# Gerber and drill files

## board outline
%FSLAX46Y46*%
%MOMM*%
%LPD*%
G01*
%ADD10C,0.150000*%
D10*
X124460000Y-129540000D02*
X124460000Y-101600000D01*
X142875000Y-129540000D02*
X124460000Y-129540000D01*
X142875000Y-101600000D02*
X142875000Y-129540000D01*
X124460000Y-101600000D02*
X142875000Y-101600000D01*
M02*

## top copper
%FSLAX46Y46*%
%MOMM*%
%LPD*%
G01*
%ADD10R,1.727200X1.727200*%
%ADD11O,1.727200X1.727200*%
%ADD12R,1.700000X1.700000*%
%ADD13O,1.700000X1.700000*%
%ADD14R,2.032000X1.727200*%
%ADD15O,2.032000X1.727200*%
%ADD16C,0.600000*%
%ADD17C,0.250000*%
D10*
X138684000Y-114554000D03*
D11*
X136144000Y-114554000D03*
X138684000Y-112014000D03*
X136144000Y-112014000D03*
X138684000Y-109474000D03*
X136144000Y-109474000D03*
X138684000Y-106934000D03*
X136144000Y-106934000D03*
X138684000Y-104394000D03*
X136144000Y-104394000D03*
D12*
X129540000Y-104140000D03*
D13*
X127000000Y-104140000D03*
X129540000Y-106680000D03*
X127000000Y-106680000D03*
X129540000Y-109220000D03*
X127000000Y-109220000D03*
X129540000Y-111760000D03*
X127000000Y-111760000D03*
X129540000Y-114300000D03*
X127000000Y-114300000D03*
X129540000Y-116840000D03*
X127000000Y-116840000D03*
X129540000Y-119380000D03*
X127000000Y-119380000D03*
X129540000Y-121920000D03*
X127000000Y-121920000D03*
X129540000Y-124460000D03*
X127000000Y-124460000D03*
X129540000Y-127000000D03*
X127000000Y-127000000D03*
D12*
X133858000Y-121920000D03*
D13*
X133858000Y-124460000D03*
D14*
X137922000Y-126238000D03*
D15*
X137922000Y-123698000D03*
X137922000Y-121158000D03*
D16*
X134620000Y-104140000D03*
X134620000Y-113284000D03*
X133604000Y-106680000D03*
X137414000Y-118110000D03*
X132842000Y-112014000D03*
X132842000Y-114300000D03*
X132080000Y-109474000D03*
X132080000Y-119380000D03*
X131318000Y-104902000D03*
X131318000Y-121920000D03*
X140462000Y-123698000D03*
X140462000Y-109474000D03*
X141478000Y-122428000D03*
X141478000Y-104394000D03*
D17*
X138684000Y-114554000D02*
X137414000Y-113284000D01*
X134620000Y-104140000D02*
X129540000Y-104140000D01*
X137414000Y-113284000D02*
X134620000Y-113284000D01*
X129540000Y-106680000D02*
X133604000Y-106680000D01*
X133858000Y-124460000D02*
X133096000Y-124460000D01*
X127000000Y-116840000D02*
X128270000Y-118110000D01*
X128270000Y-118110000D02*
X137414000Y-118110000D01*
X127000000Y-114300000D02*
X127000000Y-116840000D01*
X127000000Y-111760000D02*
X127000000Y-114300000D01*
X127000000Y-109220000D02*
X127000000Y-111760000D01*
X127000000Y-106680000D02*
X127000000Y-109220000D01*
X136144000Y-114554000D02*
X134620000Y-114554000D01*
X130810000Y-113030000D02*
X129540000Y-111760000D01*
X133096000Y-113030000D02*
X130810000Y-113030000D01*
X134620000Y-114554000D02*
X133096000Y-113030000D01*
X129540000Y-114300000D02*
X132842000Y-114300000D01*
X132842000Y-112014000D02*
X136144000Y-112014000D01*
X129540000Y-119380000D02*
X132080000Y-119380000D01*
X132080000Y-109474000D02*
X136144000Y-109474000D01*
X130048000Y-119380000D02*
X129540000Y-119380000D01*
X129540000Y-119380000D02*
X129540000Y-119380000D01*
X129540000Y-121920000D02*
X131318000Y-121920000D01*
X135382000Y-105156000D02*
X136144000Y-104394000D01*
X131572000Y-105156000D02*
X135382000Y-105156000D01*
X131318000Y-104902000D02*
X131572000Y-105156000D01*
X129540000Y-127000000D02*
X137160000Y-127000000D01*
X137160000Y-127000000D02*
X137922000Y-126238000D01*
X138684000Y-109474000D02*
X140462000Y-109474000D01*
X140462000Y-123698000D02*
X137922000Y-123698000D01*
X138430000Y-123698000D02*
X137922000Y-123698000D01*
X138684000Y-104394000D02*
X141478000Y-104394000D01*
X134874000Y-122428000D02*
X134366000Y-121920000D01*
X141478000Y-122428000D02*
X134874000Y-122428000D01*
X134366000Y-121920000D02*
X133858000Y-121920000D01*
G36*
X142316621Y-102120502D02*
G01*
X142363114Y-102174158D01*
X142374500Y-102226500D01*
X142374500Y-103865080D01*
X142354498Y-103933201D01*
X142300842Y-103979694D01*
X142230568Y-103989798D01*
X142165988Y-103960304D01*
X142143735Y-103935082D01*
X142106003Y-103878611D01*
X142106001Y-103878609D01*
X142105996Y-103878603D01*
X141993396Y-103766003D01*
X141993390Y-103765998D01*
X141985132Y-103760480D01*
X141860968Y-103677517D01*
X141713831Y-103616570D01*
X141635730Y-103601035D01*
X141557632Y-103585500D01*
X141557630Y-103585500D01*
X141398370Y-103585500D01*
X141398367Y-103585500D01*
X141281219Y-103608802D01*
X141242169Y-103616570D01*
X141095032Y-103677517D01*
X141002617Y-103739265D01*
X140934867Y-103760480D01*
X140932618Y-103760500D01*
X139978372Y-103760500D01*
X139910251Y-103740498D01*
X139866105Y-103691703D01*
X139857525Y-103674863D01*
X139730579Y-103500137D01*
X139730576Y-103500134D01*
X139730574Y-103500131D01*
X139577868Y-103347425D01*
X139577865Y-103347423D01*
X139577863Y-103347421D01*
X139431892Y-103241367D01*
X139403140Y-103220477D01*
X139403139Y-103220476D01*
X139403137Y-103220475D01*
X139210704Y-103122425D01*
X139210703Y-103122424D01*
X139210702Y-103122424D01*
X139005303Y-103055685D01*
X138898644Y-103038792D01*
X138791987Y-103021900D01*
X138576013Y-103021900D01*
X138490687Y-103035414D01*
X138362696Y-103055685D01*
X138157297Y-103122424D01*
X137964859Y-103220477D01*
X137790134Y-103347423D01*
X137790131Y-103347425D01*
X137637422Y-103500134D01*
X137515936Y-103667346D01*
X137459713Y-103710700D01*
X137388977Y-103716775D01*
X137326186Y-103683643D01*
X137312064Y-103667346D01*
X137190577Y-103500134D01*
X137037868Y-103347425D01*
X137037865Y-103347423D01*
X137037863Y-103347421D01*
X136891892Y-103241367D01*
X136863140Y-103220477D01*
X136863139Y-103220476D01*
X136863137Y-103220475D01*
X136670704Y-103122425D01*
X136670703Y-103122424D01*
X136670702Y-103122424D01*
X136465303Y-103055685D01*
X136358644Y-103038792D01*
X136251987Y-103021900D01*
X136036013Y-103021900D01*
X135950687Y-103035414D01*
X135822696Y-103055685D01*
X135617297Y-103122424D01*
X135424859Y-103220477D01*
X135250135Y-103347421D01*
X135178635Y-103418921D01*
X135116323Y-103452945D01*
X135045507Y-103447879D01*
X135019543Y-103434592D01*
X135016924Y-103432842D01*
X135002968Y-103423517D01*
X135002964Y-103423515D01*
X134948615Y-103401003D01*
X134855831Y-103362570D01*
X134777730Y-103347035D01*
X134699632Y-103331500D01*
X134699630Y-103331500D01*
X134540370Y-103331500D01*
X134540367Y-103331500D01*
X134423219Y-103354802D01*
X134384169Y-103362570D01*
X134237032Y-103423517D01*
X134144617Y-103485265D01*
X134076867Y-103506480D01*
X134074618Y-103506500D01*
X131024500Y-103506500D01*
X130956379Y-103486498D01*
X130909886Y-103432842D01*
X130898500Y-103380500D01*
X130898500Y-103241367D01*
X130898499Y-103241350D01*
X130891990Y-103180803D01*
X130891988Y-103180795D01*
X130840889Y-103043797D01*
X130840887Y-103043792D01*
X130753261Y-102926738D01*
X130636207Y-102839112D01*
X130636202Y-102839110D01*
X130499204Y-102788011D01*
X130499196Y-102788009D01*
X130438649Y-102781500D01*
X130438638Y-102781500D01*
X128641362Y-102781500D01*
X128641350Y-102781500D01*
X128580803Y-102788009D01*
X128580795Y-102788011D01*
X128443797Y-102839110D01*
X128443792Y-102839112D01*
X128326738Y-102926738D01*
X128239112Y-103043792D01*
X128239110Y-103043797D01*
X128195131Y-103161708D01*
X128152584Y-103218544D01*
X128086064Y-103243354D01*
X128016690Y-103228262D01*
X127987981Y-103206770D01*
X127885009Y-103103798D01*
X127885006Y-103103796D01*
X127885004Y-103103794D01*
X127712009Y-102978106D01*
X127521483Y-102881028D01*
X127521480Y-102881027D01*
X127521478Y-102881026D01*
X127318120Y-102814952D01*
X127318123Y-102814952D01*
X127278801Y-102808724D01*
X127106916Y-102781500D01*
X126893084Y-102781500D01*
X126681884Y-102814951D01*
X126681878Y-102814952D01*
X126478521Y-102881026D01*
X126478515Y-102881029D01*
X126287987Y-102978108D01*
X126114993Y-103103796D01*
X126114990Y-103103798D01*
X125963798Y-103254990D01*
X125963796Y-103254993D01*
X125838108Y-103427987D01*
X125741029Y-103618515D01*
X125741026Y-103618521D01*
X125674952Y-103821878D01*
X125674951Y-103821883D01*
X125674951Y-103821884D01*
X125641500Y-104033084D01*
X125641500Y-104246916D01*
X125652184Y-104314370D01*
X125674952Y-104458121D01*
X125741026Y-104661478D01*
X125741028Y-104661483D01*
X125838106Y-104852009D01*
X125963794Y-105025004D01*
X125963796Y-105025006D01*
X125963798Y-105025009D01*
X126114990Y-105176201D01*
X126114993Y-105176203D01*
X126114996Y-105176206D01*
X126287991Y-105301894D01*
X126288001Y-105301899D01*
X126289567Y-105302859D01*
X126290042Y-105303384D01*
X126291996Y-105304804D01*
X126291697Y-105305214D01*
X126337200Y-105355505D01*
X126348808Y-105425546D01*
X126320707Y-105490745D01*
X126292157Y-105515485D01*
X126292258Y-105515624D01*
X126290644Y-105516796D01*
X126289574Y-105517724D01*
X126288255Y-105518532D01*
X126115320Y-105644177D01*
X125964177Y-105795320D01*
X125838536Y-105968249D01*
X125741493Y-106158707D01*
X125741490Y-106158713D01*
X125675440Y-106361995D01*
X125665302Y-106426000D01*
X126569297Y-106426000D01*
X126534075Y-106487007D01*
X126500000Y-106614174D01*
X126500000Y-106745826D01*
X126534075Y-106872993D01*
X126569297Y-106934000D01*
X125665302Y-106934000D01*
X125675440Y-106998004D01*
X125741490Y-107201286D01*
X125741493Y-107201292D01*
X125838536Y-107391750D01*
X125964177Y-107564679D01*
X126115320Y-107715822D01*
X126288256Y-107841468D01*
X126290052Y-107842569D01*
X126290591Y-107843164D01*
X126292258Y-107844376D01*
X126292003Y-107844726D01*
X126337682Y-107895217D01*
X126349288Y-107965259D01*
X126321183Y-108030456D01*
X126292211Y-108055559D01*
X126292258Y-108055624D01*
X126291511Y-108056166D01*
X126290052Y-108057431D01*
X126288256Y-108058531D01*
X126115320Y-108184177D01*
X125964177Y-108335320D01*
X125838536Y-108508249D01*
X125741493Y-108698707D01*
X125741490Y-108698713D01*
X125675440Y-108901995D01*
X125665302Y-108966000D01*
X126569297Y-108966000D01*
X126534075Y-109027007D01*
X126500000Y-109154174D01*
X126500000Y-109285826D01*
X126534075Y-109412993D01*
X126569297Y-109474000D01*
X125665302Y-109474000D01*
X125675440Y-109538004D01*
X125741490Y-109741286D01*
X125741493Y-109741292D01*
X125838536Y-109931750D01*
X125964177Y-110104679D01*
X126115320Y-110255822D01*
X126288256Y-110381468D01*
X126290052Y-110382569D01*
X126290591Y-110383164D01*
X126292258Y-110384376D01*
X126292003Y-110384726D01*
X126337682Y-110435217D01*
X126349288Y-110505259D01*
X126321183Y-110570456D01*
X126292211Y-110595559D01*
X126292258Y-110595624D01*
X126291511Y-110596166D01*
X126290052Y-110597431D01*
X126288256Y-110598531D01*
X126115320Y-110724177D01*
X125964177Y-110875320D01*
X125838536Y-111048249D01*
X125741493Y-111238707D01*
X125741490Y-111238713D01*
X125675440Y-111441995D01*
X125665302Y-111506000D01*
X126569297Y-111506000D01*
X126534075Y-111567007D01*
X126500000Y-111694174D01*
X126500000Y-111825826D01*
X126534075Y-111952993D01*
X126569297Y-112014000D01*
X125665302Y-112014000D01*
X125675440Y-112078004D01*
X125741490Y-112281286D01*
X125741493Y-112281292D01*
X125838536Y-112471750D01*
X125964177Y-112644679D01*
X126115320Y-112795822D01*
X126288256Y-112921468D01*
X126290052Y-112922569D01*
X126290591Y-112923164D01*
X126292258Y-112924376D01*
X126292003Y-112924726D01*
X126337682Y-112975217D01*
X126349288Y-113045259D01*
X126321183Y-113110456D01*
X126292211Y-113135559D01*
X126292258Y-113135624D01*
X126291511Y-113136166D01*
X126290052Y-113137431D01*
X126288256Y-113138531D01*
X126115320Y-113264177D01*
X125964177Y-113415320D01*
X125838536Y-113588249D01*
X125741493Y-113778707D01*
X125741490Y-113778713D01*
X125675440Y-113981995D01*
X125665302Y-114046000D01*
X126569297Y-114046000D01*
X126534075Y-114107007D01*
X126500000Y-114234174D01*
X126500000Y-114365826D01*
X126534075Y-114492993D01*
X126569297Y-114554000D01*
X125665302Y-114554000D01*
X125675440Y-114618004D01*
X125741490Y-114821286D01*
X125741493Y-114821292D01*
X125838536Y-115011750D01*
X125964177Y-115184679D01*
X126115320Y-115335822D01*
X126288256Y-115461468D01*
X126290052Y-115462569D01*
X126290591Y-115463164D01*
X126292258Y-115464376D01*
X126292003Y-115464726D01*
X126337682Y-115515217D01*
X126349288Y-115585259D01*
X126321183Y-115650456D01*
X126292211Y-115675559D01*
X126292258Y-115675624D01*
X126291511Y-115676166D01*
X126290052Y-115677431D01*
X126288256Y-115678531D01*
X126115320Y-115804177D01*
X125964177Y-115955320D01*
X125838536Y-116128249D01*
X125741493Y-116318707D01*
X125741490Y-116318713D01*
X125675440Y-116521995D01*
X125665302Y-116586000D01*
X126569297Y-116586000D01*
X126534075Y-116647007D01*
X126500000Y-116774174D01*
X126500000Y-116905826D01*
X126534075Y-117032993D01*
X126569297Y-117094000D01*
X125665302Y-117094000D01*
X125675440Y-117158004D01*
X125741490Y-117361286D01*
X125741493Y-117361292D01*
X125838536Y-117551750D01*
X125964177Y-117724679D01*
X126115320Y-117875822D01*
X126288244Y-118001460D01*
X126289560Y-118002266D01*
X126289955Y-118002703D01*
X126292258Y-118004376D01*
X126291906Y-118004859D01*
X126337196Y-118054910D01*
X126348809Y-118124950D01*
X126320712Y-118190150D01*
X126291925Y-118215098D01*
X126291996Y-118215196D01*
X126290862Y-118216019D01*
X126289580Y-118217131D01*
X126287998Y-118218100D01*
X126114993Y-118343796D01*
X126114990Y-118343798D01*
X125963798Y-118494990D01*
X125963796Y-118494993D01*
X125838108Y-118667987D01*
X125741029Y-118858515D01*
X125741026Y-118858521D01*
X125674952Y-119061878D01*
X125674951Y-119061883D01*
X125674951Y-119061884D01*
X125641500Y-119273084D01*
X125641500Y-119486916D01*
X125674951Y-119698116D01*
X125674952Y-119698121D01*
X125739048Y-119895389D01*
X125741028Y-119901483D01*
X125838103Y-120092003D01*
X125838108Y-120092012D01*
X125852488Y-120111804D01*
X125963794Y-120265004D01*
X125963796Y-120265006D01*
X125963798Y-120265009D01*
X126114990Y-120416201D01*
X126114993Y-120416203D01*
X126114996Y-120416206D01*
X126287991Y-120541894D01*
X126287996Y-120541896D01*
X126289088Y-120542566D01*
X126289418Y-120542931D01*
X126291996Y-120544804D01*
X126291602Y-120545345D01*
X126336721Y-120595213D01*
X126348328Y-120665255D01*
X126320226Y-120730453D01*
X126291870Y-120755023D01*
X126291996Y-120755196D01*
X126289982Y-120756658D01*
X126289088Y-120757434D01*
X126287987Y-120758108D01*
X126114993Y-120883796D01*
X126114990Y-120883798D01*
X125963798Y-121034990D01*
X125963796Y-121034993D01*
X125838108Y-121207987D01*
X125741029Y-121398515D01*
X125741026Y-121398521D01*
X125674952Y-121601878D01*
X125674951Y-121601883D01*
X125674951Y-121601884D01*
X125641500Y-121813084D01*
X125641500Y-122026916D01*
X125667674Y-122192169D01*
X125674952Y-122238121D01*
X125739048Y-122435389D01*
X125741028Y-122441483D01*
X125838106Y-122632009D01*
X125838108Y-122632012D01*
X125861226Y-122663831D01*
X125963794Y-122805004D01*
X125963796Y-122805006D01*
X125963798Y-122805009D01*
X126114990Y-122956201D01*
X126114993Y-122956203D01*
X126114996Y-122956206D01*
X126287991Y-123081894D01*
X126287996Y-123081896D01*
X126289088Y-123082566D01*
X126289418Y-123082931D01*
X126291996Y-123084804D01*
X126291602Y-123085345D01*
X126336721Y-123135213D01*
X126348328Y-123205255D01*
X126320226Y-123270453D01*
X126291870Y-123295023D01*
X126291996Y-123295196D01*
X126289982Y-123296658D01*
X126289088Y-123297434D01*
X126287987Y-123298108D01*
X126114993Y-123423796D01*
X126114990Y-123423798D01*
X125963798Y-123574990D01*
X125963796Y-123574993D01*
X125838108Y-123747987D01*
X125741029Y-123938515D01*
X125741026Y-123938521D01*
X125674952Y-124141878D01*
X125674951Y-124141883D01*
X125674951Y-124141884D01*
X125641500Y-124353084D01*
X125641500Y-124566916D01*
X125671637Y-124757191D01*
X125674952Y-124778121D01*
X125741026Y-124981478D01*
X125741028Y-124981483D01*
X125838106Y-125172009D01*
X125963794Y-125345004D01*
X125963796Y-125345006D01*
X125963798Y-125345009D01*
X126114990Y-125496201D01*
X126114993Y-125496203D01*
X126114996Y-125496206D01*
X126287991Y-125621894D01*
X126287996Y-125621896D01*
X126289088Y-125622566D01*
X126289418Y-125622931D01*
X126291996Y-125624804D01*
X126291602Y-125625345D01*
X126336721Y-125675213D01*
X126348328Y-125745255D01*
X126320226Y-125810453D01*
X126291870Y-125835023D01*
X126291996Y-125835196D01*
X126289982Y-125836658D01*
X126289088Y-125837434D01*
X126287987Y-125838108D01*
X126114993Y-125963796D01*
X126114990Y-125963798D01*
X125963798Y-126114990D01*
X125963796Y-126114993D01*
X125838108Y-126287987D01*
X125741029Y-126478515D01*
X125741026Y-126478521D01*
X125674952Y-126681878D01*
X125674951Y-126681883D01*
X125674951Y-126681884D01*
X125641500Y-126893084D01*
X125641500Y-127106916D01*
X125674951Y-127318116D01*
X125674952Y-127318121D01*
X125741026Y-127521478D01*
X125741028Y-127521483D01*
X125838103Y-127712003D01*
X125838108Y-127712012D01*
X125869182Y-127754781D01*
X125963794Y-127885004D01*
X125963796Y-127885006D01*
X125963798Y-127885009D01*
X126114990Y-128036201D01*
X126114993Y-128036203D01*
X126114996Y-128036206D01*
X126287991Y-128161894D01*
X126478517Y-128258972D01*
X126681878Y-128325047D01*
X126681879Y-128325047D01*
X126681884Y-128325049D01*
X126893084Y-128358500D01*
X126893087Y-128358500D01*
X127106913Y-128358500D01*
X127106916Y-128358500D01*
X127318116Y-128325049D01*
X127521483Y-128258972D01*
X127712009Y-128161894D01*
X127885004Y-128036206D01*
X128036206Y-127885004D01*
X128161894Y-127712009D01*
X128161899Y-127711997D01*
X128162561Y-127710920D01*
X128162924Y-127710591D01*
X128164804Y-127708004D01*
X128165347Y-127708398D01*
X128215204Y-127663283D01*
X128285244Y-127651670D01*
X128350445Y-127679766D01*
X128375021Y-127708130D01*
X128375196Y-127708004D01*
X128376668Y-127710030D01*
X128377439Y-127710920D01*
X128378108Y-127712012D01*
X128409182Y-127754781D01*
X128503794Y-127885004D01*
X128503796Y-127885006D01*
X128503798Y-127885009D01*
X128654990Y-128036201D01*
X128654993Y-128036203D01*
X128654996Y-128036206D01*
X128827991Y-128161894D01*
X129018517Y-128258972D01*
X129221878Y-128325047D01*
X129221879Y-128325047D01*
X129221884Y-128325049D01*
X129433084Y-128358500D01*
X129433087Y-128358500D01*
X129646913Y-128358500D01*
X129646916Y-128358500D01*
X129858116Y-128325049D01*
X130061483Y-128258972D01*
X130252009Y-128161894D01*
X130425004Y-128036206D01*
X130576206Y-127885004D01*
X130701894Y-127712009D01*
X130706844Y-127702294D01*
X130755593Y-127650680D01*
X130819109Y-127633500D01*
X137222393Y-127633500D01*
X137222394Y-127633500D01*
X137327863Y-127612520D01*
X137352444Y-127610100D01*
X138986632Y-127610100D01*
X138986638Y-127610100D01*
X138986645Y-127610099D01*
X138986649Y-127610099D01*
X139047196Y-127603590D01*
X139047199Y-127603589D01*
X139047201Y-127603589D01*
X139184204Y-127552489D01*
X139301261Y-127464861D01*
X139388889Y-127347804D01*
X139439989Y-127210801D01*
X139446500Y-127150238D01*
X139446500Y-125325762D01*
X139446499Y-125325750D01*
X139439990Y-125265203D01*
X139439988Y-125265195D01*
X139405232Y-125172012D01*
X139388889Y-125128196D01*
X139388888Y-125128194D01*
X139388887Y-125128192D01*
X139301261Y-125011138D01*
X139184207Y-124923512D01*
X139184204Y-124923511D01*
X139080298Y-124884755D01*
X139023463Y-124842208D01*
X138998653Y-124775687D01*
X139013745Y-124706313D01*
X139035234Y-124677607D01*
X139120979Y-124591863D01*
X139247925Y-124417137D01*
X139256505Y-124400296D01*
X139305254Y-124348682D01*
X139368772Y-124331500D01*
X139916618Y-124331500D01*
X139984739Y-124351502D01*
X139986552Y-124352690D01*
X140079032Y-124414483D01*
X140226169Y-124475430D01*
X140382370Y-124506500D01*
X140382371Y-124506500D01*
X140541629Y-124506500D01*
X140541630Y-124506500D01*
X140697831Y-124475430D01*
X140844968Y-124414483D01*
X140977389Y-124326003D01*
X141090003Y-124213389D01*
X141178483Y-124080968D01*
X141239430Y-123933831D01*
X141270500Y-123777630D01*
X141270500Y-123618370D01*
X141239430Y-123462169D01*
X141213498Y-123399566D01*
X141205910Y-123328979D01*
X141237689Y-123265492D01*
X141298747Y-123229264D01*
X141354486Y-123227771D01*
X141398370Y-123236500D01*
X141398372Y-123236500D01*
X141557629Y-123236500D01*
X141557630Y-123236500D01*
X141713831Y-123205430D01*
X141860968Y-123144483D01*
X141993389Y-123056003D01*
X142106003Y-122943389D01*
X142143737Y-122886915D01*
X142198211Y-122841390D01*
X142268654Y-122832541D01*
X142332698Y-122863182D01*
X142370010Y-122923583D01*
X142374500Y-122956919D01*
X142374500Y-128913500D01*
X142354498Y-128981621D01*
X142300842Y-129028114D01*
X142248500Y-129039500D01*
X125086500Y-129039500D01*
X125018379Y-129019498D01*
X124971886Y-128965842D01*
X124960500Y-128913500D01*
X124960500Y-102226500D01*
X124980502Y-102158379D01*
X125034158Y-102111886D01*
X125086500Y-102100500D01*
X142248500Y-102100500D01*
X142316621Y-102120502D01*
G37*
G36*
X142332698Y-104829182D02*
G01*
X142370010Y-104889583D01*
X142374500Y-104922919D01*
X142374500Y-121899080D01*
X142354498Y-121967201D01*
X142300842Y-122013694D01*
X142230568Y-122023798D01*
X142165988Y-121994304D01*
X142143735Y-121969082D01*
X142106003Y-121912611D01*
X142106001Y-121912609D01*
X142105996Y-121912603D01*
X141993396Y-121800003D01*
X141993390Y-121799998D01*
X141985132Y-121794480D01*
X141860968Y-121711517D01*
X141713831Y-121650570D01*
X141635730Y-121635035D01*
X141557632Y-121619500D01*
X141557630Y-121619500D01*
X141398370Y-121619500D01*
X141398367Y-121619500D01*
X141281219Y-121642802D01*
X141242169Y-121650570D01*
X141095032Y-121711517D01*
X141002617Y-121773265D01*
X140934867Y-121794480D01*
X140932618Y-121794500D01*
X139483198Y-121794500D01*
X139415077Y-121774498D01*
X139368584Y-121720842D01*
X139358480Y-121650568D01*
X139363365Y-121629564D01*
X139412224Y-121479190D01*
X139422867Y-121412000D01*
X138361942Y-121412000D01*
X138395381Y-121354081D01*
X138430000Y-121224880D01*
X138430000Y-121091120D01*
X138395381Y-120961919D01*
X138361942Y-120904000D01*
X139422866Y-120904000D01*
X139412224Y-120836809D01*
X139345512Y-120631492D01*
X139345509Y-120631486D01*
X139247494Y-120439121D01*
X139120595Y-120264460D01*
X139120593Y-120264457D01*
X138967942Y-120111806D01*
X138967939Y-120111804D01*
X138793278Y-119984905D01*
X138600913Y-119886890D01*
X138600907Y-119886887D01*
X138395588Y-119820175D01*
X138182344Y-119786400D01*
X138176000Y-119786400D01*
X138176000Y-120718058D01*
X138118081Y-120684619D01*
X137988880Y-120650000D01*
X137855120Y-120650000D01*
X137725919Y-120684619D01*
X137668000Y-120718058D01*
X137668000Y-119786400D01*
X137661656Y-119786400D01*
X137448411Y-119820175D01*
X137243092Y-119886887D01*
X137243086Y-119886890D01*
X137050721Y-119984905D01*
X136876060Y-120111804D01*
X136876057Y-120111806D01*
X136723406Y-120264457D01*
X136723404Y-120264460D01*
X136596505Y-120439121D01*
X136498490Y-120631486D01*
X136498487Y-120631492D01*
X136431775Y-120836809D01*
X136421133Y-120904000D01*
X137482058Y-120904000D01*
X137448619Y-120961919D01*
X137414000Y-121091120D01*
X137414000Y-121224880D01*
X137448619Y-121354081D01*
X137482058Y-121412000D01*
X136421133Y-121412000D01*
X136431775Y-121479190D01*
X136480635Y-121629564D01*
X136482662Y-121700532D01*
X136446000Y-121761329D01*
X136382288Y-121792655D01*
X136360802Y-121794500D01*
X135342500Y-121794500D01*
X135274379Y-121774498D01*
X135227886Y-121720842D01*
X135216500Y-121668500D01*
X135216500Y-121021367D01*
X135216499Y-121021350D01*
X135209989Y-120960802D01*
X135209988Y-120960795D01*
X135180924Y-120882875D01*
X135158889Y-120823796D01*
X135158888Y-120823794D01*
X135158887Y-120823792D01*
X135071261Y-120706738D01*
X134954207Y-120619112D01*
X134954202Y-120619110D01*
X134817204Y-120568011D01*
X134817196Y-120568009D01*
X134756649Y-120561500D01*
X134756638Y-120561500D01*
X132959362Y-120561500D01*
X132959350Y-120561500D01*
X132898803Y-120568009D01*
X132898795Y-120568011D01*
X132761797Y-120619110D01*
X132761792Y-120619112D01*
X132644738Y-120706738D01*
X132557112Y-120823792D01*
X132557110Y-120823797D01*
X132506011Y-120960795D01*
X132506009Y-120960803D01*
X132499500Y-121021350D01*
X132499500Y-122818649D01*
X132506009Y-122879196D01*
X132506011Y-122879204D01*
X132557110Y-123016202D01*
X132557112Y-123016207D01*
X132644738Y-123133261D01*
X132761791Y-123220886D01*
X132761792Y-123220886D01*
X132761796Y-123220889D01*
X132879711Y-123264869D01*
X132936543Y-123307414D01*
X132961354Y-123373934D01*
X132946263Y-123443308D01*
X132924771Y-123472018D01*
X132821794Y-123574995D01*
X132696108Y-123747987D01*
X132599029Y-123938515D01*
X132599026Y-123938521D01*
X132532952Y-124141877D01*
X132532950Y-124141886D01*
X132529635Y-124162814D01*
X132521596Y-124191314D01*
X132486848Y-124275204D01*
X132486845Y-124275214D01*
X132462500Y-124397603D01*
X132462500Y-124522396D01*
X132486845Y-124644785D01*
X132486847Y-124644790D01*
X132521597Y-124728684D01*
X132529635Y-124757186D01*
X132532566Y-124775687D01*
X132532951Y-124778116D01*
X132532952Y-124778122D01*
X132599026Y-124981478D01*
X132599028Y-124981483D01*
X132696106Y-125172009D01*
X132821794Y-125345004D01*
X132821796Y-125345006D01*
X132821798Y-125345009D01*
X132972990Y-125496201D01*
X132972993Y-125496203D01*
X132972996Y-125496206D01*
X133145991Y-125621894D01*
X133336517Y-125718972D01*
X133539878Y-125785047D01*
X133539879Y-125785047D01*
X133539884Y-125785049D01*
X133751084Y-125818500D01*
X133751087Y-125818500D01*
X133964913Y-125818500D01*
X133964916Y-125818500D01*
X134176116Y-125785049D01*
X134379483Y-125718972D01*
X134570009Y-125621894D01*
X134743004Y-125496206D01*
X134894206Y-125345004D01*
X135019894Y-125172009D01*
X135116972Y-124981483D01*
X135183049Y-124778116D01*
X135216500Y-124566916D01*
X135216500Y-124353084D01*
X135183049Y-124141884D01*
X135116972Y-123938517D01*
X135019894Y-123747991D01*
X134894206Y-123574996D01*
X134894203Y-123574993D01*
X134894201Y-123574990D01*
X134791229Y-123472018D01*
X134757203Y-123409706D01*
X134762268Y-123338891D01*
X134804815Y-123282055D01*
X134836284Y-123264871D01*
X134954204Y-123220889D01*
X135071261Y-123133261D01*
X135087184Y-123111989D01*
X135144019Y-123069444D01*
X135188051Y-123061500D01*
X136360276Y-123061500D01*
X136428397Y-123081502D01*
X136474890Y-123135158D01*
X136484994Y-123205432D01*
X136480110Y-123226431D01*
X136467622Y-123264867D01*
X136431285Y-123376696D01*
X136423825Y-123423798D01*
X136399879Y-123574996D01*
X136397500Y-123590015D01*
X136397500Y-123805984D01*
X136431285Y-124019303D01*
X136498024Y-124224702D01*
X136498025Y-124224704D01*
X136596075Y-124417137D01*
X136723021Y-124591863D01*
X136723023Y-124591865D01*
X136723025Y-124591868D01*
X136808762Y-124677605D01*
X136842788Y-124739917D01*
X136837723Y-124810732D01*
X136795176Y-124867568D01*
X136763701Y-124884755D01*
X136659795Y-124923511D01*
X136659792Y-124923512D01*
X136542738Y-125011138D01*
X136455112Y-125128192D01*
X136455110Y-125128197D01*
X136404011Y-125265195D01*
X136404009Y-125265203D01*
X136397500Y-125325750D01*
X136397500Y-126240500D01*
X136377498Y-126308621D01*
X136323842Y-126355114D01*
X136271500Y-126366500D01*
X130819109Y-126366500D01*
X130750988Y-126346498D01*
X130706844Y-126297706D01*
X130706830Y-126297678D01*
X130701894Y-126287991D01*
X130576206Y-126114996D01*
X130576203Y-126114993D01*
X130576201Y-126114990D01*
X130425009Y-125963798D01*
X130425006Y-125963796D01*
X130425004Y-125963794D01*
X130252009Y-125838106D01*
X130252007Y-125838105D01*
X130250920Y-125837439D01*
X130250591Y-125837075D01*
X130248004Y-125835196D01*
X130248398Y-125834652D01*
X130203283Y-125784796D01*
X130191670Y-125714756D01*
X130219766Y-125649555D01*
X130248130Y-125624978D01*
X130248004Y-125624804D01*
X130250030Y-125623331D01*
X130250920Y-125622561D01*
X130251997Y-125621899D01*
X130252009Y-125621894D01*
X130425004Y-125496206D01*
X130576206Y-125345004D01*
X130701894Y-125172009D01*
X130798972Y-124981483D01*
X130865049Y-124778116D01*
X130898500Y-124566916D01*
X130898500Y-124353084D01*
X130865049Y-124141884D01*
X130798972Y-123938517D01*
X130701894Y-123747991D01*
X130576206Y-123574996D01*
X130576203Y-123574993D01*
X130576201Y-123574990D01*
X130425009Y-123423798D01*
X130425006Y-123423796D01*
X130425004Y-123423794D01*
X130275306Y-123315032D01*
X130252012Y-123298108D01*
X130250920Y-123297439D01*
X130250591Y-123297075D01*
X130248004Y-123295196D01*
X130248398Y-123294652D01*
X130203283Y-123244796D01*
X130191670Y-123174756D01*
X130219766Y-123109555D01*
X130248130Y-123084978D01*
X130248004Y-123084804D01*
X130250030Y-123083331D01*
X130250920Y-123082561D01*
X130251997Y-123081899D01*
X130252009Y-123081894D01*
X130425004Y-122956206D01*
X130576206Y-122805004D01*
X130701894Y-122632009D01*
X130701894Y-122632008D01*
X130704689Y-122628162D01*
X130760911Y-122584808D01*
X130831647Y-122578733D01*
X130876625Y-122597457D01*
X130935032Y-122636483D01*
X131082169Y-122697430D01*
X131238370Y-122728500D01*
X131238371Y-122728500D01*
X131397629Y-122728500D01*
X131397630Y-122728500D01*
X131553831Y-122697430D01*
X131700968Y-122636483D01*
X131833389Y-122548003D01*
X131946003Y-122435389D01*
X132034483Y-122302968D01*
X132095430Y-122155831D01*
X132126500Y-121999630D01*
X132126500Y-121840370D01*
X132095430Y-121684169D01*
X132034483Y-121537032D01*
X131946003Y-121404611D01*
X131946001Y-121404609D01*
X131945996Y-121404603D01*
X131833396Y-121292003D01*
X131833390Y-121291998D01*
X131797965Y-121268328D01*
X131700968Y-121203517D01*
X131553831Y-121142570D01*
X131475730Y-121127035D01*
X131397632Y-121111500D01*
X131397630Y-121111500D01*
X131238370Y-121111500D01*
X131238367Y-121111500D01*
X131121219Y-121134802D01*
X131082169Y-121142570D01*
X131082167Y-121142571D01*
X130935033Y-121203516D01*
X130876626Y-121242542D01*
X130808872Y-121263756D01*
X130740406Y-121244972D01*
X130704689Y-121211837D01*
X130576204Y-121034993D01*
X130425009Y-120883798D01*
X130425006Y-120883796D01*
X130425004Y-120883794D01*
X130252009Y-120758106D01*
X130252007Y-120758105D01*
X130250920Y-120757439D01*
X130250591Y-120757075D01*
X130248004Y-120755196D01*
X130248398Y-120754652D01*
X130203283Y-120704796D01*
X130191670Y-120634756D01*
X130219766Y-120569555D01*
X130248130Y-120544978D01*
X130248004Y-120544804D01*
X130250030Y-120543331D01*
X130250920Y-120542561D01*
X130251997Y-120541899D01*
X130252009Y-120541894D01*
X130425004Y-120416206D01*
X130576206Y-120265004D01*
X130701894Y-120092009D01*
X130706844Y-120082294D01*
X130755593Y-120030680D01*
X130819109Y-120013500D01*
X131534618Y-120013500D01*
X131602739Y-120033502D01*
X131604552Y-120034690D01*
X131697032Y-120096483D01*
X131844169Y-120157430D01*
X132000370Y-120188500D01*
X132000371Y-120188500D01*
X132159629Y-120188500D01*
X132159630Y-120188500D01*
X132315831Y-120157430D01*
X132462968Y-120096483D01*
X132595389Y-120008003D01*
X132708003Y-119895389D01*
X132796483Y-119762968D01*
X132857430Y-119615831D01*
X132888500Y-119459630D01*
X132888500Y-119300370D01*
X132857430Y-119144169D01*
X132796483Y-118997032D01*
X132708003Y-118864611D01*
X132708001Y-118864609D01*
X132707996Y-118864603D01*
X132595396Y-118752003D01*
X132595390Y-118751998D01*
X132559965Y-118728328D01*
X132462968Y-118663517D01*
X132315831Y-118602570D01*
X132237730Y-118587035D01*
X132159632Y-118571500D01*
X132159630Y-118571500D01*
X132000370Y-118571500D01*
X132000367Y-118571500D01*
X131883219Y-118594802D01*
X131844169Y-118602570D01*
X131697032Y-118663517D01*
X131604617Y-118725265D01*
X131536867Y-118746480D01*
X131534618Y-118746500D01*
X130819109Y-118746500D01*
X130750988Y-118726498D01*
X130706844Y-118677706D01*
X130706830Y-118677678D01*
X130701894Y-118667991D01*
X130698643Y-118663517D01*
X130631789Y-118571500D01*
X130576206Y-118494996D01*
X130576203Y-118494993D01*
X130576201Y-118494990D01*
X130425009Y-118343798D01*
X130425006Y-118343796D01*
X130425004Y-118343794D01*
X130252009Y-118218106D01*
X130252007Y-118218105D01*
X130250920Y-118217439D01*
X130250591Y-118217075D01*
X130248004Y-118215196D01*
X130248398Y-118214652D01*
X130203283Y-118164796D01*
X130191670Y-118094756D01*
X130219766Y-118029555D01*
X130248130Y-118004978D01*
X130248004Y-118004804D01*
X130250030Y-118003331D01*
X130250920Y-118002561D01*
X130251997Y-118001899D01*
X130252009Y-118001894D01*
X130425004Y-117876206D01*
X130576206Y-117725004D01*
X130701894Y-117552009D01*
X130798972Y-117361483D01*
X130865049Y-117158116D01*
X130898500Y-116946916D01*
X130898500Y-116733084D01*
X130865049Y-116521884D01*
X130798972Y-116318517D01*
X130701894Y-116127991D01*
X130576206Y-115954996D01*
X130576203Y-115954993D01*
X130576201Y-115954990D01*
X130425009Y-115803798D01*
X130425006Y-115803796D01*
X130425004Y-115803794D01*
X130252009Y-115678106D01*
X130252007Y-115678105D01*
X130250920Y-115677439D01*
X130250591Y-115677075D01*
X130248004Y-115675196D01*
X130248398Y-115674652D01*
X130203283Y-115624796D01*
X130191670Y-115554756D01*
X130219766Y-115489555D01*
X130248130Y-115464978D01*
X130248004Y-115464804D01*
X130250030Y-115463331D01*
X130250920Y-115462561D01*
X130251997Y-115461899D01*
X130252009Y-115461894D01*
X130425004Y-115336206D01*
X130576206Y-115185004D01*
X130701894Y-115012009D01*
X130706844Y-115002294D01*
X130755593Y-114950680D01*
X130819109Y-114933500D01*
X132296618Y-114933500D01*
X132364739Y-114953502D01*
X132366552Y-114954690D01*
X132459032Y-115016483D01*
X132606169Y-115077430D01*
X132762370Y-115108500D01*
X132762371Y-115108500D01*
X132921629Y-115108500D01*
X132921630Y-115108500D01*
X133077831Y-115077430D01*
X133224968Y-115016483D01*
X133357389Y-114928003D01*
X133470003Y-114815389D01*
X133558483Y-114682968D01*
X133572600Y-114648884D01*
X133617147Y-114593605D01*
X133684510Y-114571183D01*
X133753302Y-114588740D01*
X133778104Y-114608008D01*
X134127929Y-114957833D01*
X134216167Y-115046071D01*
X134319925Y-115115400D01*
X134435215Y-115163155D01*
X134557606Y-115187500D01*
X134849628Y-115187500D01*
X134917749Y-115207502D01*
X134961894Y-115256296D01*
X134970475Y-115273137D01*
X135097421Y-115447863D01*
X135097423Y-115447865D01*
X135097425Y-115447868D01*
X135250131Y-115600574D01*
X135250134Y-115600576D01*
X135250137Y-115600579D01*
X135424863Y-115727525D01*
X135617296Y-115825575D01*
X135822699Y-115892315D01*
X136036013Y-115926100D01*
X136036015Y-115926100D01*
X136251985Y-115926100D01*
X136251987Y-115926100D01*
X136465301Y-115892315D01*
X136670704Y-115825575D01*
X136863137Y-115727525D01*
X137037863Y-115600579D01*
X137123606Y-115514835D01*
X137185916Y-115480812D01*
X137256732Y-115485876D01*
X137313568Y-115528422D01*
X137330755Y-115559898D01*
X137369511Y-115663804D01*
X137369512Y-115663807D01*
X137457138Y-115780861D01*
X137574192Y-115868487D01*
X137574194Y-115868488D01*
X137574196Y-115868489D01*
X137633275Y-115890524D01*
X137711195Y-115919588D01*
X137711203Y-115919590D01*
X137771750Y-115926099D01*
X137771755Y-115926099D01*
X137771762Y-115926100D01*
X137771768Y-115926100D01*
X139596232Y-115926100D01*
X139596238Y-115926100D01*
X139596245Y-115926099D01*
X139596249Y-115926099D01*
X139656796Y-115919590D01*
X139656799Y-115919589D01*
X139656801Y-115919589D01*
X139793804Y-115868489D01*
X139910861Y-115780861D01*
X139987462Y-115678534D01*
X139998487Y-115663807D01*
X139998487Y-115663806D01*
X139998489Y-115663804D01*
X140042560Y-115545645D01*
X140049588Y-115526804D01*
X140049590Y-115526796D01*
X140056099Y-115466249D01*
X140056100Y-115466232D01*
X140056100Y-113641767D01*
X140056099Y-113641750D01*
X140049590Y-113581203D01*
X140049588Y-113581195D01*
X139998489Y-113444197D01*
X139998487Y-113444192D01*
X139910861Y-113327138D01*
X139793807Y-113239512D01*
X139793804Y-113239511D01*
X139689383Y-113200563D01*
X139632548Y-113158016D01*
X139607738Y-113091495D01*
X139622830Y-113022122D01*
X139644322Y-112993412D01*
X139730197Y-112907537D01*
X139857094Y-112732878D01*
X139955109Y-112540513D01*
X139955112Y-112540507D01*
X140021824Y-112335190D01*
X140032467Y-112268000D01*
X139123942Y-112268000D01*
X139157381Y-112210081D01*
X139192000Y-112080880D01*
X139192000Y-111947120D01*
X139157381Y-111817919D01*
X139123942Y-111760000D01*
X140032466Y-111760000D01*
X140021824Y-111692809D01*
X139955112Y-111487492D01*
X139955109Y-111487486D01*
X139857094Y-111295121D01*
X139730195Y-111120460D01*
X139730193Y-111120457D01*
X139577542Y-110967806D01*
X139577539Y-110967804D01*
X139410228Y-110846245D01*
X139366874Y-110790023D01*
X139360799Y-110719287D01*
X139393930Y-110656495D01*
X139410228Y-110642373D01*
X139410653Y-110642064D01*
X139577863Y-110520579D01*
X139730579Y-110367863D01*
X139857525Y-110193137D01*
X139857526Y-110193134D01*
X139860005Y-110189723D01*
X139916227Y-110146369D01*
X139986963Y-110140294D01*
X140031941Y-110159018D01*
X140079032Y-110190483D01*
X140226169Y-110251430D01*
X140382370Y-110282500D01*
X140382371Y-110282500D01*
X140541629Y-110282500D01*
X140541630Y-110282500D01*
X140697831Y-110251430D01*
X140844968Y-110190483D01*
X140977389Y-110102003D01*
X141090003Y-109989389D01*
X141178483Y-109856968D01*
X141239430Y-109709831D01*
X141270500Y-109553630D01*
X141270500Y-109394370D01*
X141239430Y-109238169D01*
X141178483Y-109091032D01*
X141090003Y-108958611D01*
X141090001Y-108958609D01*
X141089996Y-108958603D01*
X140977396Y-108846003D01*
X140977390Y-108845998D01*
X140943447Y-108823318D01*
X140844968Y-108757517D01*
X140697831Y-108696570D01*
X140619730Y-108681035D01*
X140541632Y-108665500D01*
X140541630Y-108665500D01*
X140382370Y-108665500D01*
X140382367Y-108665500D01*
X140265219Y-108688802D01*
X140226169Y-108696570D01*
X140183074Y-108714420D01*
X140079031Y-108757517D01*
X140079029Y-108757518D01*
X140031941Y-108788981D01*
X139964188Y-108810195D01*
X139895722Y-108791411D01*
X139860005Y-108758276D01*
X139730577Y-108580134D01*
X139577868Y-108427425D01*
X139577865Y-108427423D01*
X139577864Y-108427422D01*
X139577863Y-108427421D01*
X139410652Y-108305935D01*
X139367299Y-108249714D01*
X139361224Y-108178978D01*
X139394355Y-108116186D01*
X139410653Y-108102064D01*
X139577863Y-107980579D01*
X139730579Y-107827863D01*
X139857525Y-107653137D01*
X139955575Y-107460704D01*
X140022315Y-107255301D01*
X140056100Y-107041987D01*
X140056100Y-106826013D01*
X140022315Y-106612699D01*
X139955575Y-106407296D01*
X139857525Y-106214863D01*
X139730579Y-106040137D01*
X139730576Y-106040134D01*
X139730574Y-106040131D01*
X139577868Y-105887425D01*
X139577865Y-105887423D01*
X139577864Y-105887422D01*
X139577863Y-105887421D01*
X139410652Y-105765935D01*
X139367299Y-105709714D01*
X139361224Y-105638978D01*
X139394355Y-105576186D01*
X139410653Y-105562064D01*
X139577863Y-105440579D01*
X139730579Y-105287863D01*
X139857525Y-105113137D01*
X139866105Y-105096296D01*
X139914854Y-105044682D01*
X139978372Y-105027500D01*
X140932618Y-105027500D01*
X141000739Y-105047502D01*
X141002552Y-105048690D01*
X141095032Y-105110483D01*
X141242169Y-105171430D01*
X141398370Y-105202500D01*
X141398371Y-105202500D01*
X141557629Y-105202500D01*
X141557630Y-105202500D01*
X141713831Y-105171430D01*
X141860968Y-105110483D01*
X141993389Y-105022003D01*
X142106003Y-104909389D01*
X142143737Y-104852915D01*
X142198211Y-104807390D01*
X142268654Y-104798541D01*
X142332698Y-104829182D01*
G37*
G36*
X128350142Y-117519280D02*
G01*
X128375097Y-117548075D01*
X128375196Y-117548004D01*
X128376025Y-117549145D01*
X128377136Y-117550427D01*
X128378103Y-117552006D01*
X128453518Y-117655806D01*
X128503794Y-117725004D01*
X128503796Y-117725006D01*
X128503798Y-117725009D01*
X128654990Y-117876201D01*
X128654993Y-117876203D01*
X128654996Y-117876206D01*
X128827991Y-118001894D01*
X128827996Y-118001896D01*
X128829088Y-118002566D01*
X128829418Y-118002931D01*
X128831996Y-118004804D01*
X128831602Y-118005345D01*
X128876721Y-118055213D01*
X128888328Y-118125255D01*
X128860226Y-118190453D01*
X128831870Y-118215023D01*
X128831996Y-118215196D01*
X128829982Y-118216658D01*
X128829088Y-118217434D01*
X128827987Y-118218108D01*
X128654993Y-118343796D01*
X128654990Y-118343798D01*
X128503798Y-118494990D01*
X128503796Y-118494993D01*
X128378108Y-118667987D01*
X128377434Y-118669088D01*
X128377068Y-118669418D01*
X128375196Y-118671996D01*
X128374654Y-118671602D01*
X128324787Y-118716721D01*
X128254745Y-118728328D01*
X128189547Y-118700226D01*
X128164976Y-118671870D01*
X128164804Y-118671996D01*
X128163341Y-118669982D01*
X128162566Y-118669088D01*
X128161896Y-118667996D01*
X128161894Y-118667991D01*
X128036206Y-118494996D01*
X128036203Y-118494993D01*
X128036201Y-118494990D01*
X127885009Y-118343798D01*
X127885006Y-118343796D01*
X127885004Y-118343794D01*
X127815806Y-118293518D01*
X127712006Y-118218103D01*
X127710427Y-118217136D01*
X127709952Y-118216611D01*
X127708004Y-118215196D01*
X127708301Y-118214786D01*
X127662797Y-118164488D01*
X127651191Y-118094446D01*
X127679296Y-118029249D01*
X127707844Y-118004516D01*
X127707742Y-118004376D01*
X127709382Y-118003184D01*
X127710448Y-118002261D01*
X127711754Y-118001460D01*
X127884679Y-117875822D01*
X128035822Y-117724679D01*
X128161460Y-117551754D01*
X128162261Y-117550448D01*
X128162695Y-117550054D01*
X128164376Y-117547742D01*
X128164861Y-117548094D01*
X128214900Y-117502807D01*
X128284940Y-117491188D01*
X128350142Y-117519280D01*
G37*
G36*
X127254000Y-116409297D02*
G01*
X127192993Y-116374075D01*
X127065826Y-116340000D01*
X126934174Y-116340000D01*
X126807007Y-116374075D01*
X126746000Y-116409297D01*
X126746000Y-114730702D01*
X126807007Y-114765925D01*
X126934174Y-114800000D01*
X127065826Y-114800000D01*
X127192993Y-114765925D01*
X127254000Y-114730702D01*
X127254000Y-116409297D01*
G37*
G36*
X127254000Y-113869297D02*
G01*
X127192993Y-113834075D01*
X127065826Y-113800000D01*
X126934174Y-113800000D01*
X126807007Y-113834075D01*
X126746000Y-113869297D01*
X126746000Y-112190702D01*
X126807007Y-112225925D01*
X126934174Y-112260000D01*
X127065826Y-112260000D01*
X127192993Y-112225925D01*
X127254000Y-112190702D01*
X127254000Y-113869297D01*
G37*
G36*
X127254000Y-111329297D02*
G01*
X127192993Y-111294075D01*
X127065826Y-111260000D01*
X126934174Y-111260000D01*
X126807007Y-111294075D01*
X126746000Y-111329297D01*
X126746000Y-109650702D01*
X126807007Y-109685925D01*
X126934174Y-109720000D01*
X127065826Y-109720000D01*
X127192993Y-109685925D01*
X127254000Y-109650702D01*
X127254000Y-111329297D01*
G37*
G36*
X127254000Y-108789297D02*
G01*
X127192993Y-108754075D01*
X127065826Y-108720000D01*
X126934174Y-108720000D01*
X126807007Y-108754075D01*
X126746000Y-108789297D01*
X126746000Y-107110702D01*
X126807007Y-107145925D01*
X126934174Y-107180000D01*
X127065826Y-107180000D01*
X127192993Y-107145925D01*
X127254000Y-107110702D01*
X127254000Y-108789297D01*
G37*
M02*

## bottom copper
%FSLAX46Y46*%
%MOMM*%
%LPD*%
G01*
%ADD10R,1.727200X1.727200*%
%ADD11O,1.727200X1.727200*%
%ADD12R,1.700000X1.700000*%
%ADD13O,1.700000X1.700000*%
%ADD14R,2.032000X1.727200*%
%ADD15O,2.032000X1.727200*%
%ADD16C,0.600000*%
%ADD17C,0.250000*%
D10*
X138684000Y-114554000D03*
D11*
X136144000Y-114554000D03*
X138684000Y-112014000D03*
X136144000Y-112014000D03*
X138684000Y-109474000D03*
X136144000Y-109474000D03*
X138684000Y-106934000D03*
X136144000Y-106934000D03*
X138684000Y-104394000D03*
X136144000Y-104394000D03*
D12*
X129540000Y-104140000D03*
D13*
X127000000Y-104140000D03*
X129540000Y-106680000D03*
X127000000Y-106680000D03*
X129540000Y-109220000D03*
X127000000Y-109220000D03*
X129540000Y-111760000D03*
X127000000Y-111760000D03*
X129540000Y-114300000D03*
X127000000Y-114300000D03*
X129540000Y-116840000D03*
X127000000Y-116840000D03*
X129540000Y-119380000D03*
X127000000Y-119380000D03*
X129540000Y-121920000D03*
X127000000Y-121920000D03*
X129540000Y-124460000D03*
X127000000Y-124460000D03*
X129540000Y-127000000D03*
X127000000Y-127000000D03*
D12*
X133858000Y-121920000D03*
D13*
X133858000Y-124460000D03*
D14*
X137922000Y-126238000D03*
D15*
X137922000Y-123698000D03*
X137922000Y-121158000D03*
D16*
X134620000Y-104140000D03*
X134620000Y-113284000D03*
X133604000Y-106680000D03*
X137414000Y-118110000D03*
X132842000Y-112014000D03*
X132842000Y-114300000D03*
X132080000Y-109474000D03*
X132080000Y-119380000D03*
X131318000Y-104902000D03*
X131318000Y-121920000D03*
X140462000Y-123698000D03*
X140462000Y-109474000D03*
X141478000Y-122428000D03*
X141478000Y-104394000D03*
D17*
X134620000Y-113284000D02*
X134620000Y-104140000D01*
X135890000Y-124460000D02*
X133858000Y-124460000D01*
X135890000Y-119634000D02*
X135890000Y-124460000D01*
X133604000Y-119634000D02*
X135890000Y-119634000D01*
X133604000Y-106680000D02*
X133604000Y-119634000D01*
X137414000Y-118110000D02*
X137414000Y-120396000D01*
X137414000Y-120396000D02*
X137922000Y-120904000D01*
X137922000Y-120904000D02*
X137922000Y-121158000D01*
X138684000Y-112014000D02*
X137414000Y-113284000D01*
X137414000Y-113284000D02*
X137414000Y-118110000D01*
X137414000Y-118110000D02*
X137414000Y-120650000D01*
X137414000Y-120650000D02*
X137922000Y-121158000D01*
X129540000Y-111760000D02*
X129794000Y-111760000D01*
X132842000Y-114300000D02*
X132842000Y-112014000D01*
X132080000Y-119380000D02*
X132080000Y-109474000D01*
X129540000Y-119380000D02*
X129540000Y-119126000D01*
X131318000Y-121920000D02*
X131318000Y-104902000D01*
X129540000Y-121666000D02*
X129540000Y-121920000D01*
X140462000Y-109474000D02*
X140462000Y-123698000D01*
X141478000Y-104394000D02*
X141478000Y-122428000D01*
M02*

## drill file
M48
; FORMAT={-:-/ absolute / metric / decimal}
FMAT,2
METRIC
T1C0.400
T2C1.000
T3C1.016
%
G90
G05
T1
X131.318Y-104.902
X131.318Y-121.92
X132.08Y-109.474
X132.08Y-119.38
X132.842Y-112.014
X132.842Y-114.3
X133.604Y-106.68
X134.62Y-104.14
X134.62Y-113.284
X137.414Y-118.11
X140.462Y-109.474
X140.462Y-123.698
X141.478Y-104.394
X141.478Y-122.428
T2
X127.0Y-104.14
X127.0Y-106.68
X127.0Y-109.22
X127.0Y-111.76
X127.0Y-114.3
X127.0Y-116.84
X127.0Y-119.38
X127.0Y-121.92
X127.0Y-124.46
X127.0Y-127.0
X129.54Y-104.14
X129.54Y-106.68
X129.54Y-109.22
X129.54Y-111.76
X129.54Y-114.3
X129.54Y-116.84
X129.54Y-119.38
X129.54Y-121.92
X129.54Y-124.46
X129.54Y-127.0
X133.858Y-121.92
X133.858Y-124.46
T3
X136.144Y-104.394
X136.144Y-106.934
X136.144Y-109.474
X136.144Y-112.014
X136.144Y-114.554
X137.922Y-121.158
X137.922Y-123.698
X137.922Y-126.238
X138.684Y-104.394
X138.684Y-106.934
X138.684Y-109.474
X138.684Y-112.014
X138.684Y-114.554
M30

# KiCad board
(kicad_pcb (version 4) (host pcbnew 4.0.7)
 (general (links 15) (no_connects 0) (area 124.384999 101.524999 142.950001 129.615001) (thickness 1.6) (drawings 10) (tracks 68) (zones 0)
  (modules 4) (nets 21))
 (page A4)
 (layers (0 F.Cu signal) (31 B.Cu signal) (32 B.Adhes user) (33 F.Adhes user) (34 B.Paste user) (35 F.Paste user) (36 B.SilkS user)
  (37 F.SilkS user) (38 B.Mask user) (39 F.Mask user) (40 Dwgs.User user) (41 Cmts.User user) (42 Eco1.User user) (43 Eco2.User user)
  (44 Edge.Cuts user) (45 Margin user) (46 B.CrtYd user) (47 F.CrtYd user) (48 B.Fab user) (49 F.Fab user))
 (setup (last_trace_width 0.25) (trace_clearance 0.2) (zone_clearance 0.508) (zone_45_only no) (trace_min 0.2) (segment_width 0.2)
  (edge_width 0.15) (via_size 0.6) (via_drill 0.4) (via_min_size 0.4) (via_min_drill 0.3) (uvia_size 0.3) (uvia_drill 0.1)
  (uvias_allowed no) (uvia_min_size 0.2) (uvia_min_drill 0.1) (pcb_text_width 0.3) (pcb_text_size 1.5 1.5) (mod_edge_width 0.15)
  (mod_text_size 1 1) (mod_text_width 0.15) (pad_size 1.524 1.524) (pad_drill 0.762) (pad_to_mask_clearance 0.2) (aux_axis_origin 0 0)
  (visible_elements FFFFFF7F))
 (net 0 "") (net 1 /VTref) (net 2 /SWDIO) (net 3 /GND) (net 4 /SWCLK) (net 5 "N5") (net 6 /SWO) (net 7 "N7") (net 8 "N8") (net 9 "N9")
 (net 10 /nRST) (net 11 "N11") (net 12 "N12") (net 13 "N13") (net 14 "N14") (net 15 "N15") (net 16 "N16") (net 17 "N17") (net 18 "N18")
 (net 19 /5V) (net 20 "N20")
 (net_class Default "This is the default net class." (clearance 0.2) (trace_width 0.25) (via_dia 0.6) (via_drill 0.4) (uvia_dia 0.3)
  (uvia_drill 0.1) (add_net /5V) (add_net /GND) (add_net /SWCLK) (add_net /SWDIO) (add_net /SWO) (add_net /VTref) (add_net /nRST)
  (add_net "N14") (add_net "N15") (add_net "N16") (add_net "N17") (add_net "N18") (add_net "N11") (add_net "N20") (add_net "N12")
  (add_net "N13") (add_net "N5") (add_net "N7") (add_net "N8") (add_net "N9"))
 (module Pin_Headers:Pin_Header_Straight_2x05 (layer F.Cu) (at 138.684 114.554 180)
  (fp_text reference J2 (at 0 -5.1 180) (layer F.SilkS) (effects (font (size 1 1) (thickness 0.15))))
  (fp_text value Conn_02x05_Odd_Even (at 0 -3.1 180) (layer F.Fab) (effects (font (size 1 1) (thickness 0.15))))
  (pad 1 thru_hole rect (at 0 0 180) (size 1.7272 1.7272) (drill 1.016) (layers *.Cu *.Mask) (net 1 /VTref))
  (pad 2 thru_hole oval (at 2.54 0 180) (size 1.7272 1.7272) (drill 1.016) (layers *.Cu *.Mask) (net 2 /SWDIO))
  (pad 3 thru_hole oval (at 0 2.54 180) (size 1.7272 1.7272) (drill 1.016) (layers *.Cu *.Mask) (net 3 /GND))
  (pad 4 thru_hole oval (at 2.54 2.54 180) (size 1.7272 1.7272) (drill 1.016) (layers *.Cu *.Mask) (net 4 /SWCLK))
  (pad 5 thru_hole oval (at 0 5.08 180) (size 1.7272 1.7272) (drill 1.016) (layers *.Cu *.Mask) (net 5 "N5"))
  (pad 6 thru_hole oval (at 2.54 5.08 180) (size 1.7272 1.7272) (drill 1.016) (layers *.Cu *.Mask) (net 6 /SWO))
  (pad 7 thru_hole oval (at 0 7.62 180) (size 1.7272 1.7272) (drill 1.016) (layers *.Cu *.Mask) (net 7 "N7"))
  (pad 8 thru_hole oval (at 2.54 7.62 180) (size 1.7272 1.7272) (drill 1.016) (layers *.Cu *.Mask) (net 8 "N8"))
  (pad 9 thru_hole oval (at 0 10.16 180) (size 1.7272 1.7272) (drill 1.016) (layers *.Cu *.Mask) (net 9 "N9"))
  (pad 10 thru_hole oval (at 2.54 10.16 180) (size 1.7272 1.7272) (drill 1.016) (layers *.Cu *.Mask) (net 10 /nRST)))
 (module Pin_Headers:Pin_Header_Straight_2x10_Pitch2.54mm (layer B.Cu) (at 129.54 104.14 180)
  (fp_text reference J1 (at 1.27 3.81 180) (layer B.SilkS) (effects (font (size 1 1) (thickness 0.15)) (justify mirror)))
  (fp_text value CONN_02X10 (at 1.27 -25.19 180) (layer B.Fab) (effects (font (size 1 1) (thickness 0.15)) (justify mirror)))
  (pad 1 thru_hole rect (at 0 0 180) (size 1.7 1.7) (drill 1) (layers *.Cu *.Mask) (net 1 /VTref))
  (pad 2 thru_hole oval (at 2.54 0 180) (size 1.7 1.7) (drill 1) (layers *.Cu *.Mask) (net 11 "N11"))
  (pad 3 thru_hole oval (at 0 -2.54 180) (size 1.7 1.7) (drill 1) (layers *.Cu *.Mask) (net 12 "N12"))
  (pad 4 thru_hole oval (at 2.54 -2.54 180) (size 1.7 1.7) (drill 1) (layers *.Cu *.Mask) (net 3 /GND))
  (pad 5 thru_hole oval (at 0 -5.08 180) (size 1.7 1.7) (drill 1) (layers *.Cu *.Mask) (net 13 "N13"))
  (pad 6 thru_hole oval (at 2.54 -5.08 180) (size 1.7 1.7) (drill 1) (layers *.Cu *.Mask) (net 3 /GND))
  (pad 7 thru_hole oval (at 0 -7.62 180) (size 1.7 1.7) (drill 1) (layers *.Cu *.Mask) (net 2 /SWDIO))
  (pad 8 thru_hole oval (at 2.54 -7.62 180) (size 1.7 1.7) (drill 1) (layers *.Cu *.Mask) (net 3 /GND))
  (pad 9 thru_hole oval (at 0 -10.16 180) (size 1.7 1.7) (drill 1) (layers *.Cu *.Mask) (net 4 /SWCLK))
  (pad 10 thru_hole oval (at 2.54 -10.16 180) (size 1.7 1.7) (drill 1) (layers *.Cu *.Mask) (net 3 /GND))
  (pad 11 thru_hole oval (at 0 -12.7 180) (size 1.7 1.7) (drill 1) (layers *.Cu *.Mask) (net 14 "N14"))
  (pad 12 thru_hole oval (at 2.54 -12.7 180) (size 1.7 1.7) (drill 1) (layers *.Cu *.Mask) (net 3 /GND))
  (pad 13 thru_hole oval (at 0 -15.24 180) (size 1.7 1.7) (drill 1) (layers *.Cu *.Mask) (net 6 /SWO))
  (pad 14 thru_hole oval (at 2.54 -15.24 180) (size 1.7 1.7) (drill 1) (layers *.Cu *.Mask) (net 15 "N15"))
  (pad 15 thru_hole oval (at 0 -17.78 180) (size 1.7 1.7) (drill 1) (layers *.Cu *.Mask) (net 10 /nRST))
  (pad 16 thru_hole oval (at 2.54 -17.78 180) (size 1.7 1.7) (drill 1) (layers *.Cu *.Mask) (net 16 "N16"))
  (pad 17 thru_hole oval (at 0 -20.32 180) (size 1.7 1.7) (drill 1) (layers *.Cu *.Mask) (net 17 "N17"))
  (pad 18 thru_hole oval (at 2.54 -20.32 180) (size 1.7 1.7) (drill 1) (layers *.Cu *.Mask) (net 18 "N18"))
  (pad 19 thru_hole oval (at 0 -22.86 180) (size 1.7 1.7) (drill 1) (layers *.Cu *.Mask) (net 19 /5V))
  (pad 20 thru_hole oval (at 2.54 -22.86 180) (size 1.7 1.7) (drill 1) (layers *.Cu *.Mask) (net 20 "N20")))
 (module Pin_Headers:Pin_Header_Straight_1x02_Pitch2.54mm (layer F.Cu) (at 133.858 121.92)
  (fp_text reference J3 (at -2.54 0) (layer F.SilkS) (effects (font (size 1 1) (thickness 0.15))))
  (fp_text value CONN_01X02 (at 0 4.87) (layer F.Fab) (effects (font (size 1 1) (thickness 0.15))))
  (pad 1 thru_hole rect (at 0 0) (size 1.7 1.7) (drill 1) (layers *.Cu *.Mask) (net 9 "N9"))
  (pad 2 thru_hole oval (at 0 2.54) (size 1.7 1.7) (drill 1) (layers *.Cu *.Mask) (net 12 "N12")))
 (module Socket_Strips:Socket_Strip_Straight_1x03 (layer F.Cu) (at 137.922 126.238 90)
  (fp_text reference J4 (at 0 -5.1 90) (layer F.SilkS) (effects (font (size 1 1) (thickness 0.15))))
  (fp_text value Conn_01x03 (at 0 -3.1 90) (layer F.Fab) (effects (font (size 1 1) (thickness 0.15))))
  (pad 1 thru_hole rect (at 0 0 90) (size 1.7272 2.032) (drill 1.016) (layers *.Cu *.Mask) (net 19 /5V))
  (pad 2 thru_hole oval (at 2.54 0 90) (size 1.7272 2.032) (drill 1.016) (layers *.Cu *.Mask) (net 5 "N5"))
  (pad 3 thru_hole oval (at 5.08 0 90) (size 1.7272 2.032) (drill 1.016) (layers *.Cu *.Mask) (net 3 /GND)))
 (gr_line (start 124.46 129.54) (end 124.46 101.6) (angle 90) (layer Edge.Cuts) (width 0.15))
 (gr_line (start 142.875 129.54) (end 124.46 129.54) (angle 90) (layer Edge.Cuts) (width 0.15))
 (gr_line (start 142.875 101.6) (end 142.875 129.54) (angle 90) (layer Edge.Cuts) (width 0.15))
 (gr_line (start 124.46 101.6) (end 142.875 101.6) (angle 90) (layer Edge.Cuts) (width 0.15))
 (segment (start 138.684 114.554) (end 137.414 113.284) (width 0.25) (layer F.Cu) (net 1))
 (segment (start 134.62 104.14) (end 129.54 104.14) (width 0.25) (layer F.Cu) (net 1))
 (via (at 134.62 104.14) (size 0.6) (drill 0.4) (layers F.Cu B.Cu) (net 1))
 (segment (start 134.62 113.284) (end 134.62 104.14) (width 0.25) (layer B.Cu) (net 1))
 (via (at 134.62 113.284) (size 0.6) (drill 0.4) (layers F.Cu B.Cu) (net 1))
 (segment (start 137.414 113.284) (end 134.62 113.284) (width 0.25) (layer F.Cu) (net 1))
 (segment (start 129.54 106.68) (end 133.604 106.68) (width 0.25) (layer F.Cu) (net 12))
 (segment (start 135.89 124.46) (end 133.858 124.46) (width 0.25) (layer B.Cu) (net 12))
 (segment (start 135.89 119.634) (end 135.89 124.46) (width 0.25) (layer B.Cu) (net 12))
 (segment (start 133.604 119.634) (end 135.89 119.634) (width 0.25) (layer B.Cu) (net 12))
 (segment (start 133.604 106.68) (end 133.604 119.634) (width 0.25) (layer B.Cu) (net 12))
 (via (at 133.604 106.68) (size 0.6) (drill 0.4) (layers F.Cu B.Cu) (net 12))
 (segment (start 133.858 124.46) (end 133.096 124.46) (width 0.25) (layer F.Cu) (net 12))
 (segment (start 127 116.84) (end 128.27 118.11) (width 0.25) (layer F.Cu) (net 3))
 (via (at 137.414 118.11) (size 0.6) (drill 0.4) (layers F.Cu B.Cu) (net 3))
 (segment (start 128.27 118.11) (end 137.414 118.11) (width 0.25) (layer F.Cu) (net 3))
 (segment (start 137.414 118.11) (end 137.414 120.396) (width 0.25) (layer B.Cu) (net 3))
 (segment (start 137.414 120.396) (end 137.922 120.904) (width 0.25) (layer B.Cu) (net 3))
 (segment (start 137.922 120.904) (end 137.922 121.158) (width 0.25) (layer B.Cu) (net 3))
 (segment (start 138.684 112.014) (end 137.414 113.284) (width 0.25) (layer B.Cu) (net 3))
 (segment (start 137.414 113.284) (end 137.414 118.11) (width 0.25) (layer B.Cu) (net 3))
 (segment (start 137.414 118.11) (end 137.414 120.65) (width 0.25) (layer B.Cu) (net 3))
 (segment (start 137.414 120.65) (end 137.922 121.158) (width 0.25) (layer B.Cu) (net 3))
 (segment (start 127 114.3) (end 127 116.84) (width 0.25) (layer F.Cu) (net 3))
 (segment (start 127 111.76) (end 127 114.3) (width 0.25) (layer F.Cu) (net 3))
 (segment (start 127 109.22) (end 127 111.76) (width 0.25) (layer F.Cu) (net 3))
 (segment (start 127 106.68) (end 127 109.22) (width 0.25) (layer F.Cu) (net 3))
 (segment (start 136.144 114.554) (end 134.62 114.554) (width 0.25) (layer F.Cu) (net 2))
 (segment (start 130.81 113.03) (end 129.54 111.76) (width 0.25) (layer F.Cu) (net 2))
 (segment (start 133.096 113.03) (end 130.81 113.03) (width 0.25) (layer F.Cu) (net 2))
 (segment (start 134.62 114.554) (end 133.096 113.03) (width 0.25) (layer F.Cu) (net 2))
 (segment (start 129.54 111.76) (end 129.794 111.76) (width 0.25) (layer B.Cu) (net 2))
 (segment (start 129.54 114.3) (end 132.842 114.3) (width 0.25) (layer F.Cu) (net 4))
 (segment (start 132.842 112.014) (end 136.144 112.014) (width 0.25) (layer F.Cu) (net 4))
 (via (at 132.842 112.014) (size 0.6) (drill 0.4) (layers F.Cu B.Cu) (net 4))
 (segment (start 132.842 114.3) (end 132.842 112.014) (width 0.25) (layer B.Cu) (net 4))
 (via (at 132.842 114.3) (size 0.6) (drill 0.4) (layers F.Cu B.Cu) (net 4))
 (segment (start 129.54 119.38) (end 132.08 119.38) (width 0.25) (layer F.Cu) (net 6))
 (segment (start 132.08 109.474) (end 136.144 109.474) (width 0.25) (layer F.Cu) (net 6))
 (via (at 132.08 109.474) (size 0.6) (drill 0.4) (layers F.Cu B.Cu) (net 6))
 (segment (start 132.08 119.38) (end 132.08 109.474) (width 0.25) (layer B.Cu) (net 6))
 (via (at 132.08 119.38) (size 0.6) (drill 0.4) (layers F.Cu B.Cu) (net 6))
 (segment (start 130.048 119.38) (end 129.54 119.38) (width 0.25) (layer F.Cu) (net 6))
 (segment (start 129.54 119.38) (end 129.54 119.126) (width 0.25) (layer B.Cu) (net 6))
 (segment (start 129.54 119.38) (end 129.54 119.38) (width 0.25) (layer F.Cu) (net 6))
 (segment (start 129.54 121.92) (end 131.318 121.92) (width 0.25) (layer F.Cu) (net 10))
 (segment (start 135.382 105.156) (end 136.144 104.394) (width 0.25) (layer F.Cu) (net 10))
 (segment (start 131.572 105.156) (end 135.382 105.156) (width 0.25) (layer F.Cu) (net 10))
 (segment (start 131.318 104.902) (end 131.572 105.156) (width 0.25) (layer F.Cu) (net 10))
 (via (at 131.318 104.902) (size 0.6) (drill 0.4) (layers F.Cu B.Cu) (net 10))
 (segment (start 131.318 121.92) (end 131.318 104.902) (width 0.25) (layer B.Cu) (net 10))
 (via (at 131.318 121.92) (size 0.6) (drill 0.4) (layers F.Cu B.Cu) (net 10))
 (segment (start 129.54 121.666) (end 129.54 121.92) (width 0.25) (layer B.Cu) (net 10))
 (segment (start 129.54 127) (end 137.16 127) (width 0.25) (layer F.Cu) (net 19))
 (segment (start 137.16 127) (end 137.922 126.238) (width 0.25) (layer F.Cu) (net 19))
 (segment (start 138.684 109.474) (end 140.462 109.474) (width 0.25) (layer F.Cu) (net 5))
 (segment (start 140.462 123.698) (end 137.922 123.698) (width 0.25) (layer F.Cu) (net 5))
 (via (at 140.462 123.698) (size 0.6) (drill 0.4) (layers F.Cu B.Cu) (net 5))
 (segment (start 140.462 109.474) (end 140.462 123.698) (width 0.25) (layer B.Cu) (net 5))
 (via (at 140.462 109.474) (size 0.6) (drill 0.4) (layers F.Cu B.Cu) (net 5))
 (segment (start 138.43 123.698) (end 137.922 123.698) (width 0.25) (layer F.Cu) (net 5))
 (segment (start 138.684 104.394) (end 141.478 104.394) (width 0.25) (layer F.Cu) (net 9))
 (segment (start 134.874 122.428) (end 134.366 121.92) (width 0.25) (layer F.Cu) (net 9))
 (segment (start 141.478 122.428) (end 134.874 122.428) (width 0.25) (layer F.Cu) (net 9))
 (via (at 141.478 122.428) (size 0.6) (drill 0.4) (layers F.Cu B.Cu) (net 9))
 (segment (start 141.478 104.394) (end 141.478 122.428) (width 0.25) (layer B.Cu) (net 9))
 (via (at 141.478 104.394) (size 0.6) (drill 0.4) (layers F.Cu B.Cu) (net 9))
 (segment (start 134.366 121.92) (end 133.858 121.92) (width 0.25) (layer F.Cu) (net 9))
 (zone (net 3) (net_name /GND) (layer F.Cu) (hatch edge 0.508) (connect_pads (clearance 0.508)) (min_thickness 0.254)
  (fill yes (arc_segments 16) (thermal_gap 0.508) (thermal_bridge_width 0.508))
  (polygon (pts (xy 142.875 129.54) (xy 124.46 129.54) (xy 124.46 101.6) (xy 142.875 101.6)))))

